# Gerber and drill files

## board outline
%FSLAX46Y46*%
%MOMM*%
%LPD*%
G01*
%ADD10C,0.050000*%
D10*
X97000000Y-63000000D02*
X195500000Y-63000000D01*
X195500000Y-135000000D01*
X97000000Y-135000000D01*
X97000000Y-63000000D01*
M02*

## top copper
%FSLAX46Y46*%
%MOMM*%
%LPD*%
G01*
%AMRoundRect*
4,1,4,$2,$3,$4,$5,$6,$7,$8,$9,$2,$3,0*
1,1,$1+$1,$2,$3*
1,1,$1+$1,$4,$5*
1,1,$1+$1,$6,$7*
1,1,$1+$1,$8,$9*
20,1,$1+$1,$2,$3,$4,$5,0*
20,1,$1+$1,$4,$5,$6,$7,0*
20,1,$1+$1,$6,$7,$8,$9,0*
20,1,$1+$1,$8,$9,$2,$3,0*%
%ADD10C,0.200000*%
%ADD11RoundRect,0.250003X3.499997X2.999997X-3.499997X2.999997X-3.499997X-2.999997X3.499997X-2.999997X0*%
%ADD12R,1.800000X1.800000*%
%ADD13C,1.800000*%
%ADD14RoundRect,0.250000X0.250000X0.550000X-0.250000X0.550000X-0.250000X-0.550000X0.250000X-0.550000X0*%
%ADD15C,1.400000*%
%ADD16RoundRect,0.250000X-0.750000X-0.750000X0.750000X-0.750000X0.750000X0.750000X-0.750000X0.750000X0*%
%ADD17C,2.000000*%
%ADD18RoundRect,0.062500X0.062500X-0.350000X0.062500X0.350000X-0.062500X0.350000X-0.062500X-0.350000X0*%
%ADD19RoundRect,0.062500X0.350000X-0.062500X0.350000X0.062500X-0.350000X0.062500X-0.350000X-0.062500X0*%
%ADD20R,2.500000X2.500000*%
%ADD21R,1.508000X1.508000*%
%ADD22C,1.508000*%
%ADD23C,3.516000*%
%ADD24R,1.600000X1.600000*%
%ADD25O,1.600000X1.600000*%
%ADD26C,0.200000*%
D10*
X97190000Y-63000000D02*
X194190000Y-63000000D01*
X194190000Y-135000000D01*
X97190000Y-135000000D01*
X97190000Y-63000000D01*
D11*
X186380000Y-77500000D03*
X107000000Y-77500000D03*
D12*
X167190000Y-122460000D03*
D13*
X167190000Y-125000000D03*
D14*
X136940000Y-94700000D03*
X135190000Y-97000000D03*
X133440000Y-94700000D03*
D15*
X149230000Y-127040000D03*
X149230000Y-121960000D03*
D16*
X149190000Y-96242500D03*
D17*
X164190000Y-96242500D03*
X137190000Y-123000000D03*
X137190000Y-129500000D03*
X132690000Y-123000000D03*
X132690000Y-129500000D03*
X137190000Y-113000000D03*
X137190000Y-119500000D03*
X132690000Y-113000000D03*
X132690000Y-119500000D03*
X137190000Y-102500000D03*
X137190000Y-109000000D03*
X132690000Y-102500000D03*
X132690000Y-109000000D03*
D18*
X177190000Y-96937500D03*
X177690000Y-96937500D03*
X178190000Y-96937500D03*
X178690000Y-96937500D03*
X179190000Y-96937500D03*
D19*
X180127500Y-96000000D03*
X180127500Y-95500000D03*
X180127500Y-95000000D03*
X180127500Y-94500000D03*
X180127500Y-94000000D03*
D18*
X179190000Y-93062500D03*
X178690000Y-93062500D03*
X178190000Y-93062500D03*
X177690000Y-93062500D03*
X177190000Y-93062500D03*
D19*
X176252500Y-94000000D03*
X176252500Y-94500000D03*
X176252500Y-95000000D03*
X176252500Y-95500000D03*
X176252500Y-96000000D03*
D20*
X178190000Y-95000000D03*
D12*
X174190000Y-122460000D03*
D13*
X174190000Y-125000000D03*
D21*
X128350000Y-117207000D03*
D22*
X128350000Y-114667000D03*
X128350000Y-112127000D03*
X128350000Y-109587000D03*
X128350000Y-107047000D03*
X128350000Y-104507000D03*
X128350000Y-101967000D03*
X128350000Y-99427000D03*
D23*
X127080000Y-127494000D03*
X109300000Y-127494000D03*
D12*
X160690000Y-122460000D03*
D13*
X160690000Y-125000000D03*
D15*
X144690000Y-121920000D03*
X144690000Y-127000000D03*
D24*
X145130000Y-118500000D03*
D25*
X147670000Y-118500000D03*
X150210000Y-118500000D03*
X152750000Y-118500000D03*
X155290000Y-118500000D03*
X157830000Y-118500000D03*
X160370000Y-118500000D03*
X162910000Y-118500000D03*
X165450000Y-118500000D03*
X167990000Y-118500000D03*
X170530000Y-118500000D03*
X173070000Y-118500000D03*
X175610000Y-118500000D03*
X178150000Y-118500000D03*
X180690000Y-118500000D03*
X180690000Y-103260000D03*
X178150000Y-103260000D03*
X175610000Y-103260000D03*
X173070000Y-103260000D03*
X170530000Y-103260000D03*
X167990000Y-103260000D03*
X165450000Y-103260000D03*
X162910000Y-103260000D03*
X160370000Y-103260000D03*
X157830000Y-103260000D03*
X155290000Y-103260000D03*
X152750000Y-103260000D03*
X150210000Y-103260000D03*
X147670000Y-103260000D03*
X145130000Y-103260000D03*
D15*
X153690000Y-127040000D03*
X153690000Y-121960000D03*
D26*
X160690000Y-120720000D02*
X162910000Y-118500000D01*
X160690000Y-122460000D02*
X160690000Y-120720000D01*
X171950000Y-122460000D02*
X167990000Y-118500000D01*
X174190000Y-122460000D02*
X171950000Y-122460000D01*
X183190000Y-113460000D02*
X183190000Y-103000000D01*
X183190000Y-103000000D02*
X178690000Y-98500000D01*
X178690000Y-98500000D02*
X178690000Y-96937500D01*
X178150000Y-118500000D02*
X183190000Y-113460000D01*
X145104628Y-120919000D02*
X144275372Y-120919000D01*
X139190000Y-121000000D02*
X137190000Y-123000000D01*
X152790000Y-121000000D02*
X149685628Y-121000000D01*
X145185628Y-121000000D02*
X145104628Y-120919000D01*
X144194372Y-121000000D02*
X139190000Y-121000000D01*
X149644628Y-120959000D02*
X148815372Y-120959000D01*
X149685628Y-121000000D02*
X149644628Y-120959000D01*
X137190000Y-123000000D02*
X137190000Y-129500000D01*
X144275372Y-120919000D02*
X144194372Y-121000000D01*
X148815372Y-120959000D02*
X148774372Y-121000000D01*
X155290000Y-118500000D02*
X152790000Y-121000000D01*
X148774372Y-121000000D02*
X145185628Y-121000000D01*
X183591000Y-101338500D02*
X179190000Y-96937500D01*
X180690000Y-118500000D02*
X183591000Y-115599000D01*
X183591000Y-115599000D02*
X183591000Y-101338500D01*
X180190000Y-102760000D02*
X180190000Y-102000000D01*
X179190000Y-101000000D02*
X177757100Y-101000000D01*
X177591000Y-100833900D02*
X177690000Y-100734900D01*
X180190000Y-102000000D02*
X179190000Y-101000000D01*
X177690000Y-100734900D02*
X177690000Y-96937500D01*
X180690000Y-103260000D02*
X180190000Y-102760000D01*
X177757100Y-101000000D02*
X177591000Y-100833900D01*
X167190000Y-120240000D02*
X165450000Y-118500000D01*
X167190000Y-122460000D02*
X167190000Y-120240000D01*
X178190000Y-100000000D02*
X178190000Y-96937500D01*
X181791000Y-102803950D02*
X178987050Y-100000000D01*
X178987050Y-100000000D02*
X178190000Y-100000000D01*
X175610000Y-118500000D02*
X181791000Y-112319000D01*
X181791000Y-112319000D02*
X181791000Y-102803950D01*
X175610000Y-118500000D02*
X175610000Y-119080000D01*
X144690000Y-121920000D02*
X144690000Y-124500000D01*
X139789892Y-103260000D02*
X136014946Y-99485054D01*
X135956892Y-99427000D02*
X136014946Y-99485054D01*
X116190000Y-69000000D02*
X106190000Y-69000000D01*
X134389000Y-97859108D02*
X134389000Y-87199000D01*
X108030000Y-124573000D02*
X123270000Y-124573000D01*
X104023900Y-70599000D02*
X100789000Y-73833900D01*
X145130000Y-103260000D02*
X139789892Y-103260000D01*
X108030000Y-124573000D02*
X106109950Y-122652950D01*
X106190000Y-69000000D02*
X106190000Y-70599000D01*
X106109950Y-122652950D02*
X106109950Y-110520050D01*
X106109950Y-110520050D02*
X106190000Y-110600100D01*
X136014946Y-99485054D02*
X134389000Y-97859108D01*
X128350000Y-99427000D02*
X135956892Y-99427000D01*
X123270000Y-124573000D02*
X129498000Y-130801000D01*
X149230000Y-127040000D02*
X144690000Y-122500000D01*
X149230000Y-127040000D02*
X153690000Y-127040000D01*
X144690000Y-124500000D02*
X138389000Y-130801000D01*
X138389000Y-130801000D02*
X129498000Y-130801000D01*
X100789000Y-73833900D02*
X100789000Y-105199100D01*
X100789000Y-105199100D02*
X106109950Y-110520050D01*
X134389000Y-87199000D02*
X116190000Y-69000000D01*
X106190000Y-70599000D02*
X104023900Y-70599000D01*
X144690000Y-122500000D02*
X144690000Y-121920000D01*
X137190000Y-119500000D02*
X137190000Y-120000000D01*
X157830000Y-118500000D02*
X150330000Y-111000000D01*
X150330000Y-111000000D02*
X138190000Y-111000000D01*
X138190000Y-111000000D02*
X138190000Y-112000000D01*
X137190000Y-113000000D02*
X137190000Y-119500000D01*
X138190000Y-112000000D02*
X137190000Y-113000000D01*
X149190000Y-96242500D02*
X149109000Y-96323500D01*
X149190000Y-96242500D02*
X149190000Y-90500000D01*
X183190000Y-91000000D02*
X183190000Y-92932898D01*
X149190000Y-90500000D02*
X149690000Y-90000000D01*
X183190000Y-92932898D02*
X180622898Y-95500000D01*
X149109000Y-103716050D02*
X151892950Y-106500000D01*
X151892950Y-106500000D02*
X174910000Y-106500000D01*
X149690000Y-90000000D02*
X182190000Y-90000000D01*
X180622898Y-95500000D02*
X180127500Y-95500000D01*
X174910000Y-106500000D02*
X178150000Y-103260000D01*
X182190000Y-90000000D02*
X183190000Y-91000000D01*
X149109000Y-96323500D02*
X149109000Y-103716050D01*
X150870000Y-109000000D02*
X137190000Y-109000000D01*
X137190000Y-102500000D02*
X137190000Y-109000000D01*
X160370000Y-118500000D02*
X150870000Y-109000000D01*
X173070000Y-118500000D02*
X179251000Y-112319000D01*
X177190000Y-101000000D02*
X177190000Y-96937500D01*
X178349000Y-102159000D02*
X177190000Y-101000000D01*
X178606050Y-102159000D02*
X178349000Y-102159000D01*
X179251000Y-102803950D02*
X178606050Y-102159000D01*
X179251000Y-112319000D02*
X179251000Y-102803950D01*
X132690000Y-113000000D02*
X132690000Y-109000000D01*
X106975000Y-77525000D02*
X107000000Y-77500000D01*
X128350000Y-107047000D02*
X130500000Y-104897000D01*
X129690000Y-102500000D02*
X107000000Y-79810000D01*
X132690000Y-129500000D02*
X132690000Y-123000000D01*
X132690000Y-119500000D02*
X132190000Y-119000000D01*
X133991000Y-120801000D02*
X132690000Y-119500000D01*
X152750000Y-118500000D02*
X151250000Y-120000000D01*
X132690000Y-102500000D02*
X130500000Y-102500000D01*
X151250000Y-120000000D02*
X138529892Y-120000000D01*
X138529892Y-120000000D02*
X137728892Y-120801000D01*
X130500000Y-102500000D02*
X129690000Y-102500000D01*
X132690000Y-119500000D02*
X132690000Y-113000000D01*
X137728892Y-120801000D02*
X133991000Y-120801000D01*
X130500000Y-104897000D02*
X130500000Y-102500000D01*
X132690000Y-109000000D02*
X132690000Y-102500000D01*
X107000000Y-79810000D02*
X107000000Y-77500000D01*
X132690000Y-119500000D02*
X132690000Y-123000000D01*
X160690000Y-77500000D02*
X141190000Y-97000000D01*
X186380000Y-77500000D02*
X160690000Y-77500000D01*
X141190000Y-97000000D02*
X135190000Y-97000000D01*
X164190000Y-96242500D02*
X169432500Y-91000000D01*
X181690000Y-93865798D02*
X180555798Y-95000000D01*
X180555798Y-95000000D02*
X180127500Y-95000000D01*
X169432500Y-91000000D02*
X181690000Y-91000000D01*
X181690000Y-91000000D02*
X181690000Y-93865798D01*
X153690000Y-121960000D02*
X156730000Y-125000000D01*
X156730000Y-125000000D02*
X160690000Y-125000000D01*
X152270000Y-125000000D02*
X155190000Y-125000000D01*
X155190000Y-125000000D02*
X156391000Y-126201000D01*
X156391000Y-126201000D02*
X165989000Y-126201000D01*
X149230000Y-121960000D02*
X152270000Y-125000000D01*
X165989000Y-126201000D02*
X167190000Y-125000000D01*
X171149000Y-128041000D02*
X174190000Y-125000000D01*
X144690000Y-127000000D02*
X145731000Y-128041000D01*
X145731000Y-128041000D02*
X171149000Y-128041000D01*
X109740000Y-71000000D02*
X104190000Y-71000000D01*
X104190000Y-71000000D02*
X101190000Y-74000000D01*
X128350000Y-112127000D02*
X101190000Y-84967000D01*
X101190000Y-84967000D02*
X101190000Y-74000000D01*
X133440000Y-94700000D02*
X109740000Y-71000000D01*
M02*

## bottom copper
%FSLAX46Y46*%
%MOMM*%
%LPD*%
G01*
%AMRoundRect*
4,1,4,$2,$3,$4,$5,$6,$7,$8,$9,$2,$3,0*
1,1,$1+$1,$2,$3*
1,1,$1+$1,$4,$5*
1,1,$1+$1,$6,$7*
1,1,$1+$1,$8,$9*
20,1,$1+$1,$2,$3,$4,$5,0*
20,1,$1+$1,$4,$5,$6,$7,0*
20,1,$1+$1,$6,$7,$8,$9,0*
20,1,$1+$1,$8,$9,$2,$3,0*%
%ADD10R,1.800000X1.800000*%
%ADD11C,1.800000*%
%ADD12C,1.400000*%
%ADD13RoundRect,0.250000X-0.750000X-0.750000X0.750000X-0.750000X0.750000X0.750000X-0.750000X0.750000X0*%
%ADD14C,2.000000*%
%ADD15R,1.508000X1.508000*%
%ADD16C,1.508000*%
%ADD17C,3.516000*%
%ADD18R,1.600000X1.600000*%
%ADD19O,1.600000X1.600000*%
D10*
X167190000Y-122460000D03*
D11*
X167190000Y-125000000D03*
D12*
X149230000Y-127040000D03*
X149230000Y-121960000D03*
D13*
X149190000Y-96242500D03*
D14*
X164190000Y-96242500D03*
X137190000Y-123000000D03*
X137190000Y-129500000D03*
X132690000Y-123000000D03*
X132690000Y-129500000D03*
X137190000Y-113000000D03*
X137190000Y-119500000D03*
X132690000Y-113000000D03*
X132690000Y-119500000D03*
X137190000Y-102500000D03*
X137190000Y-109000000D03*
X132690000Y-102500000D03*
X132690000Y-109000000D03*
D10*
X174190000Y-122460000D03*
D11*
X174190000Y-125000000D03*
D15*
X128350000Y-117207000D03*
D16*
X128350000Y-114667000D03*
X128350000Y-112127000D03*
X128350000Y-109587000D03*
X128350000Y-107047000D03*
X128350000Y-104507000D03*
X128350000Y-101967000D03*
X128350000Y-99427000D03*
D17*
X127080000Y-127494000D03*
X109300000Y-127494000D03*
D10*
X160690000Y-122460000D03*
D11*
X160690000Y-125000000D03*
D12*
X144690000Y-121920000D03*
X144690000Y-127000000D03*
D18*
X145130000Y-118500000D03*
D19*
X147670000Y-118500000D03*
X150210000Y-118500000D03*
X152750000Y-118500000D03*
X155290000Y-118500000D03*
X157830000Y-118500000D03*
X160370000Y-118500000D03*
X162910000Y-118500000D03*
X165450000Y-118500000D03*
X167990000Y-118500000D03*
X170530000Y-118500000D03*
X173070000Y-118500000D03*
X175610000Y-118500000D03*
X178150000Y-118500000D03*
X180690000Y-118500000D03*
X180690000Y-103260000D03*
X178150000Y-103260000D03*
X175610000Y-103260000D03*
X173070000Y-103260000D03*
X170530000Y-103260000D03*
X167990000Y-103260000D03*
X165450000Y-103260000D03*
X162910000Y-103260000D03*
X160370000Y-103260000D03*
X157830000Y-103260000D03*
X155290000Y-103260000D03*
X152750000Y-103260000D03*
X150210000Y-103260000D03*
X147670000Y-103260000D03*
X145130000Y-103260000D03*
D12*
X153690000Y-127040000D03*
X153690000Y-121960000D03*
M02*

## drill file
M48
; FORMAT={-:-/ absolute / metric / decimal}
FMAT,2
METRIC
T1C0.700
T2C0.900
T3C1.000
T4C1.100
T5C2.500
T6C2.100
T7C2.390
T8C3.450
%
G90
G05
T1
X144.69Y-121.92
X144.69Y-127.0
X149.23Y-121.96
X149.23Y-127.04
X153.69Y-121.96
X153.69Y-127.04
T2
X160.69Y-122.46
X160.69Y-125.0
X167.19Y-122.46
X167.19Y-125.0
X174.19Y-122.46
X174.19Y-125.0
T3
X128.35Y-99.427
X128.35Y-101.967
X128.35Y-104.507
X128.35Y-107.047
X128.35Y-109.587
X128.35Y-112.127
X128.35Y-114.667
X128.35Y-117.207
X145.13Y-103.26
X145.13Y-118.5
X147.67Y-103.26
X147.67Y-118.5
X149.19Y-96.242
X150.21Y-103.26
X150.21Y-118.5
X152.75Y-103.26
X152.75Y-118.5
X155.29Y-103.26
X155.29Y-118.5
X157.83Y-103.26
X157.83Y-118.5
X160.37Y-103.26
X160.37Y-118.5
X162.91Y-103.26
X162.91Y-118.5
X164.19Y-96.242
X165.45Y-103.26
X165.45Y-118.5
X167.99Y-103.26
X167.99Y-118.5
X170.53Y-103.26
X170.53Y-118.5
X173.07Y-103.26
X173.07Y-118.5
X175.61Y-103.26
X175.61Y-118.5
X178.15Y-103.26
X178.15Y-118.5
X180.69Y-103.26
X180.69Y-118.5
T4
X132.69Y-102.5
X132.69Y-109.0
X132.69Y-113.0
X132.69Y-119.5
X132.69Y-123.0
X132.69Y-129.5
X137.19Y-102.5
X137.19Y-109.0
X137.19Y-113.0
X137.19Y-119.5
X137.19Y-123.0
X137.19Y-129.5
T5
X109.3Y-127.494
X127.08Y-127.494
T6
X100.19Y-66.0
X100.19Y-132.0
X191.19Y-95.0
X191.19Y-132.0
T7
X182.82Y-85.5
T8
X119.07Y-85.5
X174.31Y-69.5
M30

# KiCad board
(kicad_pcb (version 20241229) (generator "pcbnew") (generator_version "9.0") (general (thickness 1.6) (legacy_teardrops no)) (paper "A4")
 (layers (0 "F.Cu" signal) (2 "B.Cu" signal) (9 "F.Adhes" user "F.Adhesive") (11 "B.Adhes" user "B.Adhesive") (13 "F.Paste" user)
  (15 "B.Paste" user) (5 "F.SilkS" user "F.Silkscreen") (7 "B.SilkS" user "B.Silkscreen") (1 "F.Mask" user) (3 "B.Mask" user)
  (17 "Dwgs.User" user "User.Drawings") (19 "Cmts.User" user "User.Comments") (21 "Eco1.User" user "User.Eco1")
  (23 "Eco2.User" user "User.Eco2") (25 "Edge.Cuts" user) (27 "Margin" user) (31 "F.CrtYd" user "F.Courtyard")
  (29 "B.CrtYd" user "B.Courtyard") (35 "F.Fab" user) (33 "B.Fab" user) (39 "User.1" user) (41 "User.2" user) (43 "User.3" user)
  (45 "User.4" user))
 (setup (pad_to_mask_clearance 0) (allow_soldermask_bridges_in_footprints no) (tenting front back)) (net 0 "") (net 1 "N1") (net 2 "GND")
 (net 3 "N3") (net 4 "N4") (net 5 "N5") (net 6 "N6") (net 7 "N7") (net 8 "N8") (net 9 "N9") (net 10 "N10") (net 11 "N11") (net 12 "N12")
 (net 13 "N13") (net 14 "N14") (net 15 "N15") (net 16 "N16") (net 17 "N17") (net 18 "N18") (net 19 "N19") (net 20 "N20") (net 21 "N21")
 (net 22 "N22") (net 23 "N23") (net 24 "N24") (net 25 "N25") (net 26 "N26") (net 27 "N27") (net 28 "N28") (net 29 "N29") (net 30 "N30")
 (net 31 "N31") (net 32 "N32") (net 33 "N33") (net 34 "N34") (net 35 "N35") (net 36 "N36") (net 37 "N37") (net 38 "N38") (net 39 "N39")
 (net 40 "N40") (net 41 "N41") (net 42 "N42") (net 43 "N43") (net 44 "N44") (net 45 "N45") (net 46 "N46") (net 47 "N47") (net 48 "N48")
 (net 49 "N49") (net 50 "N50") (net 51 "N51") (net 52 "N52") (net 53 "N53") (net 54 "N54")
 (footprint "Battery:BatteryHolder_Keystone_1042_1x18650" (layer "F.Cu") (at 146.69 77.5 180)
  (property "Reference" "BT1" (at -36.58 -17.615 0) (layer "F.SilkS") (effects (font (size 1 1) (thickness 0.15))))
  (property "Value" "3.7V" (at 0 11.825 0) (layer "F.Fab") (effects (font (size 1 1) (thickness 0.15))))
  (pad "" np_thru_hole circle (at -36.13 -8 180) (size 2.39 2.39) (drill 2.39) (layers "*.Cu" "*.Mask"))
  (pad "" np_thru_hole circle (at -27.62 8 180) (size 3.45 3.45) (drill 3.45) (layers "*.Cu" "*.Mask"))
  (pad "" np_thru_hole circle (at 27.62 -8 180) (size 3.45 3.45) (drill 3.45) (layers "*.Cu" "*.Mask"))
  (pad "1" smd roundrect (at -39.69 0 180) (size 7.5 6.5) (layers "F.Cu" "F.Mask" "F.Paste") (roundrect_rratio 0.038462) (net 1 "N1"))
  (pad "2" smd roundrect (at 39.69 0 180) (size 7.5 6.5) (layers "F.Cu" "F.Mask" "F.Paste") (roundrect_rratio 0.038462) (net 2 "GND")))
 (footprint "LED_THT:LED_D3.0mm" (layer "F.Cu") (at 167.19 122.46 -90)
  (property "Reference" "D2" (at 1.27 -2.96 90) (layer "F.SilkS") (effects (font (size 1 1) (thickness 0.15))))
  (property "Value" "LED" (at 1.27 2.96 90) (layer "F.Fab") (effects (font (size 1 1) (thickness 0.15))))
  (pad "1" thru_hole rect (at 0 0 270) (size 1.8 1.8) (drill 0.9) (layers "*.Cu" "*.Mask") (remove_unused_layers no) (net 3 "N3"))
  (pad "2" thru_hole circle (at 2.54 0 270) (size 1.8 1.8) (drill 0.9) (layers "*.Cu" "*.Mask") (remove_unused_layers no) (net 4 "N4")))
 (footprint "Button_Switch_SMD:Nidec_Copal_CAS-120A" (layer "F.Cu") (at 135.19 95.85 -90)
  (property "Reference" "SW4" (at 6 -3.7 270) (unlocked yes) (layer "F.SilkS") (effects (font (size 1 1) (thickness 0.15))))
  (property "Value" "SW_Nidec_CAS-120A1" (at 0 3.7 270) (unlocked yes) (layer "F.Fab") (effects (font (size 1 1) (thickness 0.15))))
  (pad "1" smd roundrect (at -1.15 -1.75 180) (size 1 1.6) (layers "F.Cu" "F.Mask" "F.Paste") (roundrect_rratio 0.25) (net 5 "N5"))
  (pad "2" smd roundrect (at 1.15 0 180) (size 1 1.6) (layers "F.Cu" "F.Mask" "F.Paste") (roundrect_rratio 0.25) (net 1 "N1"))
  (pad "3" smd roundrect (at -1.15 1.75 180) (size 1 1.6) (layers "F.Cu" "F.Mask" "F.Paste") (roundrect_rratio 0.25) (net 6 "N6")))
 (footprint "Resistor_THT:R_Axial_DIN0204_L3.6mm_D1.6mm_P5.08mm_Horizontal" (layer "F.Cu") (at 149.23 127.04 90)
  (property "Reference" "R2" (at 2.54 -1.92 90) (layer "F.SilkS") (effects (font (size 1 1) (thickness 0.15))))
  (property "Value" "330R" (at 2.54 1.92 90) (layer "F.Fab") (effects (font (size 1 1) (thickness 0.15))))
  (pad "1" thru_hole circle (at 0 0 90) (size 1.4 1.4) (drill 0.7) (layers "*.Cu" "*.Mask") (remove_unused_layers no) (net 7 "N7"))
  (pad "2" thru_hole circle (at 5.08 0 90) (size 1.4 1.4) (drill 0.7) (layers "*.Cu" "*.Mask") (remove_unused_layers no) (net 4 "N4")))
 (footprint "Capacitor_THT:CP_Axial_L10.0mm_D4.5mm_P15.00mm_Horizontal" (layer "F.Cu") (at 149.19 96.2425)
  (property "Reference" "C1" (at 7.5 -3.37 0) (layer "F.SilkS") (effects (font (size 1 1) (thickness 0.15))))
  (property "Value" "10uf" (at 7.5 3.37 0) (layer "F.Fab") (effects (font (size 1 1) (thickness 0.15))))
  (pad "1" thru_hole roundrect (at 0 0) (size 2 2) (drill 1) (layers "*.Cu" "*.Mask") (remove_unused_layers no) (roundrect_rratio 0.125)
   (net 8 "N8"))
  (pad "2" thru_hole circle (at 15 0) (size 2 2) (drill 1) (layers "*.Cu" "*.Mask") (remove_unused_layers no) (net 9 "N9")))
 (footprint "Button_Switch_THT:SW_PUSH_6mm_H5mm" (layer "F.Cu") (at 137.19 123 -90)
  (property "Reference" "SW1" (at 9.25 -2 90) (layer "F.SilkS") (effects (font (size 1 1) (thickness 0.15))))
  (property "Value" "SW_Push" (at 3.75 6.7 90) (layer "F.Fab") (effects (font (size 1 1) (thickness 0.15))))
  (pad "1" thru_hole circle (at 0 0) (size 2 2) (drill 1.1) (layers "*.Cu" "*.Mask") (remove_unused_layers no) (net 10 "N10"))
  (pad "1" thru_hole circle (at 6.5 0) (size 2 2) (drill 1.1) (layers "*.Cu" "*.Mask") (remove_unused_layers no) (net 10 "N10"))
  (pad "2" thru_hole circle (at 0 4.5) (size 2 2) (drill 1.1) (layers "*.Cu" "*.Mask") (remove_unused_layers no) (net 2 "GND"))
  (pad "2" thru_hole circle (at 6.5 4.5) (size 2 2) (drill 1.1) (layers "*.Cu" "*.Mask") (remove_unused_layers no) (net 2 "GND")))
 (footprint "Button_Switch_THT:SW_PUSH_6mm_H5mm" (layer "F.Cu") (at 137.19 113 -90)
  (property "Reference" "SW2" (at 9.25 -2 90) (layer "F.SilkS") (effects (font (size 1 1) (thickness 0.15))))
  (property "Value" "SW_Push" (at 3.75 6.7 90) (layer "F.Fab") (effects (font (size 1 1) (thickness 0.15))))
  (pad "1" thru_hole circle (at 0 0) (size 2 2) (drill 1.1) (layers "*.Cu" "*.Mask") (remove_unused_layers no) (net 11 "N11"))
  (pad "1" thru_hole circle (at 6.5 0) (size 2 2) (drill 1.1) (layers "*.Cu" "*.Mask") (remove_unused_layers no) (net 11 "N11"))
  (pad "2" thru_hole circle (at 0 4.5) (size 2 2) (drill 1.1) (layers "*.Cu" "*.Mask") (remove_unused_layers no) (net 2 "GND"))
  (pad "2" thru_hole circle (at 6.5 4.5) (size 2 2) (drill 1.1) (layers "*.Cu" "*.Mask") (remove_unused_layers no) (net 2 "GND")))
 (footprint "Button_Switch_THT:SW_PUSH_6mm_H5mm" (layer "F.Cu") (at 137.19 102.5 -90)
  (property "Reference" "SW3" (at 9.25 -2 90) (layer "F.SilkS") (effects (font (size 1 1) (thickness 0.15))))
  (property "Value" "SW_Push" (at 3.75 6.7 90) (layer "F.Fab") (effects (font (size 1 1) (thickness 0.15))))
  (pad "1" thru_hole circle (at 0 0) (size 2 2) (drill 1.1) (layers "*.Cu" "*.Mask") (remove_unused_layers no) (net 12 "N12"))
  (pad "1" thru_hole circle (at 6.5 0) (size 2 2) (drill 1.1) (layers "*.Cu" "*.Mask") (remove_unused_layers no) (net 12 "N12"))
  (pad "2" thru_hole circle (at 0 4.5) (size 2 2) (drill 1.1) (layers "*.Cu" "*.Mask") (remove_unused_layers no) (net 2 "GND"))
  (pad "2" thru_hole circle (at 6.5 4.5) (size 2 2) (drill 1.1) (layers "*.Cu" "*.Mask") (remove_unused_layers no) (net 2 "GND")))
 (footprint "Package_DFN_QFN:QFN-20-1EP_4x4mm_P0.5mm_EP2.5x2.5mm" (layer "F.Cu") (at 178.19 95 90)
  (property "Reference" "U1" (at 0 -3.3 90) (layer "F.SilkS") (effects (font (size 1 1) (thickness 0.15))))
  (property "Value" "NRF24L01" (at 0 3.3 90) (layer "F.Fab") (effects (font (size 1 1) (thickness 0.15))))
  (pad "" smd roundrect (at -0.625 -0.625 90) (size 1.01 1.01) (layers "F.Paste") (roundrect_rratio 0.247525))
  (pad "" smd roundrect (at -0.625 0.625 90) (size 1.01 1.01) (layers "F.Paste") (roundrect_rratio 0.247525))
  (pad "" smd roundrect (at 0.625 -0.625 90) (size 1.01 1.01) (layers "F.Paste") (roundrect_rratio 0.247525))
  (pad "" smd roundrect (at 0.625 0.625 90) (size 1.01 1.01) (layers "F.Paste") (roundrect_rratio 0.247525))
  (pad "1" smd roundrect (at -1.9375 -1 90) (size 0.825 0.25) (layers "F.Cu" "F.Mask" "F.Paste") (roundrect_rratio 0.25) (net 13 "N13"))
  (pad "2" smd roundrect (at -1.9375 -0.5 90) (size 0.825 0.25) (layers "F.Cu" "F.Mask" "F.Paste") (roundrect_rratio 0.25) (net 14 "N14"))
  (pad "3" smd roundrect (at -1.9375 0 90) (size 0.825 0.25) (layers "F.Cu" "F.Mask" "F.Paste") (roundrect_rratio 0.25) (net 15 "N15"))
  (pad "4" smd roundrect (at -1.9375 0.5 90) (size 0.825 0.25) (layers "F.Cu" "F.Mask" "F.Paste") (roundrect_rratio 0.25) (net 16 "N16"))
  (pad "5" smd roundrect (at -1.9375 1 90) (size 0.825 0.25) (layers "F.Cu" "F.Mask" "F.Paste") (roundrect_rratio 0.25) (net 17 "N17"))
  (pad "6" smd roundrect (at -1 1.9375 90) (size 0.25 0.825) (layers "F.Cu" "F.Mask" "F.Paste") (roundrect_rratio 0.25) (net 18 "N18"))
  (pad "7" smd roundrect (at -0.5 1.9375 90) (size 0.25 0.825) (layers "F.Cu" "F.Mask" "F.Paste") (roundrect_rratio 0.25) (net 8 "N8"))
  (pad "8" smd roundrect (at 0 1.9375 90) (size 0.25 0.825) (layers "F.Cu" "F.Mask" "F.Paste") (roundrect_rratio 0.25) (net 9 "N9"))
  (pad "9" smd roundrect (at 0.5 1.9375 90) (size 0.25 0.825) (layers "F.Cu" "F.Mask" "F.Paste") (roundrect_rratio 0.25) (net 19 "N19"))
  (pad "10" smd roundrect (at 1 1.9375 90) (size 0.25 0.825) (layers "F.Cu" "F.Mask" "F.Paste") (roundrect_rratio 0.25) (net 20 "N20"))
  (pad "11" smd roundrect (at 1.9375 1 90) (size 0.825 0.25) (layers "F.Cu" "F.Mask" "F.Paste") (roundrect_rratio 0.25) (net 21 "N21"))
  (pad "12" smd roundrect (at 1.9375 0.5 90) (size 0.825 0.25) (layers "F.Cu" "F.Mask" "F.Paste") (roundrect_rratio 0.25) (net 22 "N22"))
  (pad "13" smd roundrect (at 1.9375 0 90) (size 0.825 0.25) (layers "F.Cu" "F.Mask" "F.Paste") (roundrect_rratio 0.25) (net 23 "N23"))
  (pad "14" smd roundrect (at 1.9375 -0.5 90) (size 0.825 0.25) (layers "F.Cu" "F.Mask" "F.Paste") (roundrect_rratio 0.25) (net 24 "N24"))
  (pad "15" smd roundrect (at 1.9375 -1 90) (size 0.825 0.25) (layers "F.Cu" "F.Mask" "F.Paste") (roundrect_rratio 0.25) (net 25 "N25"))
  (pad "16" smd roundrect (at 1 -1.9375 90) (size 0.25 0.825) (layers "F.Cu" "F.Mask" "F.Paste") (roundrect_rratio 0.25) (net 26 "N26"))
  (pad "17" smd roundrect (at 0.5 -1.9375 90) (size 0.25 0.825) (layers "F.Cu" "F.Mask" "F.Paste") (roundrect_rratio 0.25) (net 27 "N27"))
  (pad "18" smd roundrect (at 0 -1.9375 90) (size 0.25 0.825) (layers "F.Cu" "F.Mask" "F.Paste") (roundrect_rratio 0.25) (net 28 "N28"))
  (pad "19" smd roundrect (at -0.5 -1.9375 90) (size 0.25 0.825) (layers "F.Cu" "F.Mask" "F.Paste") (roundrect_rratio 0.25) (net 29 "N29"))
  (pad "20" smd roundrect (at -1 -1.9375 90) (size 0.25 0.825) (layers "F.Cu" "F.Mask" "F.Paste") (roundrect_rratio 0.25) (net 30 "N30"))
  (pad "21" smd rect (at 0 0 90) (size 2.5 2.5) (layers "F.Cu" "F.Mask") (zone_connect 2)))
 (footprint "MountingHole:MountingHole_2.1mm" (layer "F.Cu") (at 191.19 95 -90)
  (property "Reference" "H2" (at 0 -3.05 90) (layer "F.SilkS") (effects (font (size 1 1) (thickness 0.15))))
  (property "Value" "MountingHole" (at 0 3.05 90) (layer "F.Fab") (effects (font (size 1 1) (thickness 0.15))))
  (pad "" np_thru_hole circle (at 0 0 270) (size 2.1 2.1) (drill 2.1) (layers "*.Cu" "*.Mask")))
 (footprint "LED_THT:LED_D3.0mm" (layer "F.Cu") (at 174.19 122.46 -90)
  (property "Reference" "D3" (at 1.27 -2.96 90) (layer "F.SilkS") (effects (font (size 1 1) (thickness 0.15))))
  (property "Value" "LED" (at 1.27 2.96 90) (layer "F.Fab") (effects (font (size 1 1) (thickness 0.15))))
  (pad "1" thru_hole rect (at 0 0 270) (size 1.8 1.8) (drill 0.9) (layers "*.Cu" "*.Mask") (remove_unused_layers no) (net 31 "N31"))
  (pad "2" thru_hole circle (at 2.54 0 270) (size 1.8 1.8) (drill 0.9) (layers "*.Cu" "*.Mask") (remove_unused_layers no) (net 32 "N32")))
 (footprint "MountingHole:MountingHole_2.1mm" (layer "F.Cu") (at 100.19 66 -90)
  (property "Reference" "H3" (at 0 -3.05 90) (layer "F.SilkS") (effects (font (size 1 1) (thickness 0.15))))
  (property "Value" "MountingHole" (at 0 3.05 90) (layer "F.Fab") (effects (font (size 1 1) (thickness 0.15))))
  (pad "" np_thru_hole circle (at 0 0 270) (size 2.1 2.1) (drill 2.1) (layers "*.Cu" "*.Mask")))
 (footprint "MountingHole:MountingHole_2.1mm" (layer "F.Cu") (at 191.19 132 -90)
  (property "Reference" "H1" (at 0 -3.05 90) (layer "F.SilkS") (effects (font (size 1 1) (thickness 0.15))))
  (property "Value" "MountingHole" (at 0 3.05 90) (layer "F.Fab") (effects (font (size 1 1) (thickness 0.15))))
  (pad "" np_thru_hole circle (at 0 0 270) (size 2.1 2.1) (drill 2.1) (layers "*.Cu" "*.Mask")))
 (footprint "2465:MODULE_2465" (layer "F.Cu") (at 118.19 112 90)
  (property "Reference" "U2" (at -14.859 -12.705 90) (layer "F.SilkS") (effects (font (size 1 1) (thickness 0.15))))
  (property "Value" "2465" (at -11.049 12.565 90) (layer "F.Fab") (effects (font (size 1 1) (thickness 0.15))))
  (pad "1" thru_hole rect (at -5.207 10.16 90) (size 1.508 1.508) (drill 1) (layers "*.Cu" "*.Mask") (remove_unused_layers no)
   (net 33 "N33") (solder_mask_margin 0.102))
  (pad "2" thru_hole circle (at -2.667 10.16 90) (size 1.508 1.508) (drill 1) (layers "*.Cu" "*.Mask") (remove_unused_layers no)
   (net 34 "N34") (solder_mask_margin 0.102))
  (pad "3" thru_hole circle (at -0.127 10.16 90) (size 1.508 1.508) (drill 1) (layers "*.Cu" "*.Mask") (remove_unused_layers no)
   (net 6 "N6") (solder_mask_margin 0.102))
  (pad "4" thru_hole circle (at 2.413 10.16 90) (size 1.508 1.508) (drill 1) (layers "*.Cu" "*.Mask") (remove_unused_layers no)
   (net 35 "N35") (solder_mask_margin 0.102))
  (pad "5" thru_hole circle (at 4.953 10.16 90) (size 1.508 1.508) (drill 1) (layers "*.Cu" "*.Mask") (remove_unused_layers no)
   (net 2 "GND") (solder_mask_margin 0.102))
  (pad "6" thru_hole circle (at 7.493 10.16 90) (size 1.508 1.508) (drill 1) (layers "*.Cu" "*.Mask") (remove_unused_layers no)
   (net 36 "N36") (solder_mask_margin 0.102))
  (pad "7" thru_hole circle (at 10.033 10.16 90) (size 1.508 1.508) (drill 1) (layers "*.Cu" "*.Mask") (remove_unused_layers no)
   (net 2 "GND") (solder_mask_margin 0.102))
  (pad "8" thru_hole circle (at 12.573 10.16 90) (size 1.508 1.508) (drill 1) (layers "*.Cu" "*.Mask") (remove_unused_layers no)
   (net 7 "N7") (solder_mask_margin 0.102))
  (pad "P1" thru_hole circle (at -15.494 8.89 90) (size 3.516 3.516) (drill 2.5) (layers "*.Cu" "*.Mask") (remove_unused_layers no)
   (solder_mask_margin 0.102))
  (pad "P2" thru_hole circle (at -15.494 -8.89 90) (size 3.516 3.516) (drill 2.5) (layers "*.Cu" "*.Mask") (remove_unused_layers no)
   (solder_mask_margin 0.102)))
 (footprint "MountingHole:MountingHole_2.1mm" (layer "F.Cu") (at 100.19 132 -90)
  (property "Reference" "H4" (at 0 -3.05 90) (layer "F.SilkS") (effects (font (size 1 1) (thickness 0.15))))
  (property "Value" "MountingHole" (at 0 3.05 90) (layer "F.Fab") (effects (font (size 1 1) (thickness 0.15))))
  (pad "" np_thru_hole circle (at 0 0 270) (size 2.1 2.1) (drill 2.1) (layers "*.Cu" "*.Mask")))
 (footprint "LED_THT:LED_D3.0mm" (layer "F.Cu") (at 160.69 122.46 -90)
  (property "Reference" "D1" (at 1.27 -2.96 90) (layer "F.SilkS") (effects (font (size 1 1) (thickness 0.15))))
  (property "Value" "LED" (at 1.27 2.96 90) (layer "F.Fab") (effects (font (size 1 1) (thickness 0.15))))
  (pad "1" thru_hole rect (at 0 0 270) (size 1.8 1.8) (drill 0.9) (layers "*.Cu" "*.Mask") (remove_unused_layers no) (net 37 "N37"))
  (pad "2" thru_hole circle (at 2.54 0 270) (size 1.8 1.8) (drill 0.9) (layers "*.Cu" "*.Mask") (remove_unused_layers no) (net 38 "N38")))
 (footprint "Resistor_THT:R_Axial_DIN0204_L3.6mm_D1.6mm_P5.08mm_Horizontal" (layer "F.Cu") (at 144.69 121.92 -90)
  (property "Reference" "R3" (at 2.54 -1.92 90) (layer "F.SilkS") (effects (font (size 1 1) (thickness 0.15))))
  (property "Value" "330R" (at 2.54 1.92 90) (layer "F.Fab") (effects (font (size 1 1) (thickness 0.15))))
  (pad "1" thru_hole circle (at 0 0 270) (size 1.4 1.4) (drill 0.7) (layers "*.Cu" "*.Mask") (remove_unused_layers no) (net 7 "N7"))
  (pad "2" thru_hole circle (at 5.08 0 270) (size 1.4 1.4) (drill 0.7) (layers "*.Cu" "*.Mask") (remove_unused_layers no) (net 32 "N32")))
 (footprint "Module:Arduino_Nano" (layer "F.Cu") (at 145.13 118.5 90)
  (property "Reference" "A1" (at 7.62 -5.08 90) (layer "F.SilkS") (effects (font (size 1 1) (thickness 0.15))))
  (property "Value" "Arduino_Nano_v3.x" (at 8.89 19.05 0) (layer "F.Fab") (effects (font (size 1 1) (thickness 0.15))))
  (pad "1" thru_hole rect (at 0 0 90) (size 1.6 1.6) (drill 1) (layers "*.Cu" "*.Mask") (remove_unused_layers no) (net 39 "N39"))
  (pad "2" thru_hole oval (at 0 2.54 90) (size 1.6 1.6) (drill 1) (layers "*.Cu" "*.Mask") (remove_unused_layers no) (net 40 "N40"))
  (pad "3" thru_hole oval (at 0 5.08 90) (size 1.6 1.6) (drill 1) (layers "*.Cu" "*.Mask") (remove_unused_layers no) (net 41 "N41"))
  (pad "4" thru_hole oval (at 0 7.62 90) (size 1.6 1.6) (drill 1) (layers "*.Cu" "*.Mask") (remove_unused_layers no) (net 2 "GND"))
  (pad "5" thru_hole oval (at 0 10.16 90) (size 1.6 1.6) (drill 1) (layers "*.Cu" "*.Mask") (remove_unused_layers no) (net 10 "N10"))
  (pad "6" thru_hole oval (at 0 12.7 90) (size 1.6 1.6) (drill 1) (layers "*.Cu" "*.Mask") (remove_unused_layers no) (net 11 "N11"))
  (pad "7" thru_hole oval (at 0 15.24 90) (size 1.6 1.6) (drill 1) (layers "*.Cu" "*.Mask") (remove_unused_layers no) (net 12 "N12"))
  (pad "8" thru_hole oval (at 0 17.78 90) (size 1.6 1.6) (drill 1) (layers "*.Cu" "*.Mask") (remove_unused_layers no) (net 37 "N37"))
  (pad "9" thru_hole oval (at 0 20.32 90) (size 1.6 1.6) (drill 1) (layers "*.Cu" "*.Mask") (remove_unused_layers no) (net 3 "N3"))
  (pad "10" thru_hole oval (at 0 22.86 90) (size 1.6 1.6) (drill 1) (layers "*.Cu" "*.Mask") (remove_unused_layers no) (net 31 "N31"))
  (pad "11" thru_hole oval (at 0 25.4 90) (size 1.6 1.6) (drill 1) (layers "*.Cu" "*.Mask") (remove_unused_layers no) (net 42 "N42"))
  (pad "12" thru_hole oval (at 0 27.94 90) (size 1.6 1.6) (drill 1) (layers "*.Cu" "*.Mask") (remove_unused_layers no) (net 13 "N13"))
  (pad "13" thru_hole oval (at 0 30.48 90) (size 1.6 1.6) (drill 1) (layers "*.Cu" "*.Mask") (remove_unused_layers no) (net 15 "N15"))
  (pad "14" thru_hole oval (at 0 33.02 90) (size 1.6 1.6) (drill 1) (layers "*.Cu" "*.Mask") (remove_unused_layers no) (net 16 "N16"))
  (pad "15" thru_hole oval (at 0 35.56 90) (size 1.6 1.6) (drill 1) (layers "*.Cu" "*.Mask") (remove_unused_layers no) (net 17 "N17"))
  (pad "16" thru_hole oval (at 15.24 35.56 90) (size 1.6 1.6) (drill 1) (layers "*.Cu" "*.Mask") (remove_unused_layers no) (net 14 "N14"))
  (pad "17" thru_hole oval (at 15.24 33.02 90) (size 1.6 1.6) (drill 1) (layers "*.Cu" "*.Mask") (remove_unused_layers no) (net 8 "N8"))
  (pad "18" thru_hole oval (at 15.24 30.48 90) (size 1.6 1.6) (drill 1) (layers "*.Cu" "*.Mask") (remove_unused_layers no) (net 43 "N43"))
  (pad "19" thru_hole oval (at 15.24 27.94 90) (size 1.6 1.6) (drill 1) (layers "*.Cu" "*.Mask") (remove_unused_layers no) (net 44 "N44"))
  (pad "20" thru_hole oval (at 15.24 25.4 90) (size 1.6 1.6) (drill 1) (layers "*.Cu" "*.Mask") (remove_unused_layers no) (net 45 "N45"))
  (pad "21" thru_hole oval (at 15.24 22.86 90) (size 1.6 1.6) (drill 1) (layers "*.Cu" "*.Mask") (remove_unused_layers no) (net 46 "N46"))
  (pad "22" thru_hole oval (at 15.24 20.32 90) (size 1.6 1.6) (drill 1) (layers "*.Cu" "*.Mask") (remove_unused_layers no) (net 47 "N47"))
  (pad "23" thru_hole oval (at 15.24 17.78 90) (size 1.6 1.6) (drill 1) (layers "*.Cu" "*.Mask") (remove_unused_layers no) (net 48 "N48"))
  (pad "24" thru_hole oval (at 15.24 15.24 90) (size 1.6 1.6) (drill 1) (layers "*.Cu" "*.Mask") (remove_unused_layers no) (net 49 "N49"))
  (pad "25" thru_hole oval (at 15.24 12.7 90) (size 1.6 1.6) (drill 1) (layers "*.Cu" "*.Mask") (remove_unused_layers no) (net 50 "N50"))
  (pad "26" thru_hole oval (at 15.24 10.16 90) (size 1.6 1.6) (drill 1) (layers "*.Cu" "*.Mask") (remove_unused_layers no) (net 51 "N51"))
  (pad "27" thru_hole oval (at 15.24 7.62 90) (size 1.6 1.6) (drill 1) (layers "*.Cu" "*.Mask") (remove_unused_layers no) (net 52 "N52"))
  (pad "28" thru_hole oval (at 15.24 5.08 90) (size 1.6 1.6) (drill 1) (layers "*.Cu" "*.Mask") (remove_unused_layers no) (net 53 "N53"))
  (pad "29" thru_hole oval (at 15.24 2.54 90) (size 1.6 1.6) (drill 1) (layers "*.Cu" "*.Mask") (remove_unused_layers no) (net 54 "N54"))
  (pad "30" thru_hole oval (at 15.24 0 90) (size 1.6 1.6) (drill 1) (layers "*.Cu" "*.Mask") (remove_unused_layers no) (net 7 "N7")))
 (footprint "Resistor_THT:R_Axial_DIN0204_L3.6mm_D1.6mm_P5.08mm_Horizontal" (layer "F.Cu") (at 153.69 127.04 90)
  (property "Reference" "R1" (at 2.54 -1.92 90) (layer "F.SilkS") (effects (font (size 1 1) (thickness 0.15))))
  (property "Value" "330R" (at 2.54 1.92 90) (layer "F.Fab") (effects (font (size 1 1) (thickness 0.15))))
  (pad "1" thru_hole circle (at 0 0 90) (size 1.4 1.4) (drill 0.7) (layers "*.Cu" "*.Mask") (remove_unused_layers no) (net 7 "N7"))
  (pad "2" thru_hole circle (at 5.08 0 90) (size 1.4 1.4) (drill 0.7) (layers "*.Cu" "*.Mask") (remove_unused_layers no) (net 38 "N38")))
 (gr_rect (start 97.19 63) (end 194.19 135) (stroke (width 0.2) (type default)) (fill no) (layer "F.Cu"))
 (gr_rect (start 97 63) (end 195.5 135) (stroke (width 0.05) (type default)) (fill no) (layer "Edge.Cuts"))
 (segment (start 160.69 120.72) (end 162.91 118.5) (width 0.2) (layer "F.Cu") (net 37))
 (segment (start 160.69 122.46) (end 160.69 120.72) (width 0.2) (layer "F.Cu") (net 37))
 (segment (start 171.95 122.46) (end 167.99 118.5) (width 0.2) (layer "F.Cu") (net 31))
 (segment (start 174.19 122.46) (end 171.95 122.46) (width 0.2) (layer "F.Cu") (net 31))
 (segment (start 183.19 113.46) (end 183.19 103) (width 0.2) (layer "F.Cu") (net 16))
 (segment (start 183.19 103) (end 178.69 98.5) (width 0.2) (layer "F.Cu") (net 16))
 (segment (start 178.69 98.5) (end 178.69 96.9375) (width 0.2) (layer "F.Cu") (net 16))
 (segment (start 178.15 118.5) (end 183.19 113.46) (width 0.2) (layer "F.Cu") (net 16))
 (segment (start 145.104628 120.919) (end 144.275372 120.919) (width 0.2) (layer "F.Cu") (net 10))
 (segment (start 139.19 121) (end 137.19 123) (width 0.2) (layer "F.Cu") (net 10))
 (segment (start 152.79 121) (end 149.685628 121) (width 0.2) (layer "F.Cu") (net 10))
 (segment (start 145.185628 121) (end 145.104628 120.919) (width 0.2) (layer "F.Cu") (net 10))
 (segment (start 144.194372 121) (end 139.19 121) (width 0.2) (layer "F.Cu") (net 10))
 (segment (start 149.644628 120.959) (end 148.815372 120.959) (width 0.2) (layer "F.Cu") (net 10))
 (segment (start 149.685628 121) (end 149.644628 120.959) (width 0.2) (layer "F.Cu") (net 10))
 (segment (start 137.19 123) (end 137.19 129.5) (width 0.2) (layer "F.Cu") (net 10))
 (segment (start 144.275372 120.919) (end 144.194372 121) (width 0.2) (layer "F.Cu") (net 10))
 (segment (start 148.815372 120.959) (end 148.774372 121) (width 0.2) (layer "F.Cu") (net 10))
 (segment (start 155.29 118.5) (end 152.79 121) (width 0.2) (layer "F.Cu") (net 10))
 (segment (start 148.774372 121) (end 145.185628 121) (width 0.2) (layer "F.Cu") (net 10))
 (segment (start 183.591 101.3385) (end 179.19 96.9375) (width 0.2) (layer "F.Cu") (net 17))
 (segment (start 180.69 118.5) (end 183.591 115.599) (width 0.2) (layer "F.Cu") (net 17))
 (segment (start 183.591 115.599) (end 183.591 101.3385) (width 0.2) (layer "F.Cu") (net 17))
 (segment (start 180.19 102.76) (end 180.19 102) (width 0.2) (layer "F.Cu") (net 14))
 (segment (start 179.19 101) (end 177.7571 101) (width 0.2) (layer "F.Cu") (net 14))
 (segment (start 177.591 100.8339) (end 177.69 100.7349) (width 0.2) (layer "F.Cu") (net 14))
 (segment (start 180.19 102) (end 179.19 101) (width 0.2) (layer "F.Cu") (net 14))
 (segment (start 177.69 100.7349) (end 177.69 96.9375) (width 0.2) (layer "F.Cu") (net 14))
 (segment (start 180.69 103.26) (end 180.19 102.76) (width 0.2) (layer "F.Cu") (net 14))
 (segment (start 177.7571 101) (end 177.591 100.8339) (width 0.2) (layer "F.Cu") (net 14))
 (segment (start 167.19 120.24) (end 165.45 118.5) (width 0.2) (layer "F.Cu") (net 3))
 (segment (start 167.19 122.46) (end 167.19 120.24) (width 0.2) (layer "F.Cu") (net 3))
 (segment (start 178.19 100) (end 178.19 96.9375) (width 0.2) (layer "F.Cu") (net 15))
 (segment (start 181.791 102.80395) (end 178.98705 100) (width 0.2) (layer "F.Cu") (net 15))
 (segment (start 178.98705 100) (end 178.19 100) (width 0.2) (layer "F.Cu") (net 15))
 (segment (start 175.61 118.5) (end 181.791 112.319) (width 0.2) (layer "F.Cu") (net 15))
 (segment (start 181.791 112.319) (end 181.791 102.80395) (width 0.2) (layer "F.Cu") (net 15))
 (segment (start 175.61 118.5) (end 175.61 119.08) (width 0.2) (layer "F.Cu") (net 15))
 (segment (start 144.69 121.92) (end 144.69 124.5) (width 0.2) (layer "F.Cu") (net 7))
 (segment (start 139.789892 103.26) (end 136.014946 99.485054) (width 0.2) (layer "F.Cu") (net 7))
 (segment (start 135.956892 99.427) (end 136.014946 99.485054) (width 0.2) (layer "F.Cu") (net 7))
 (segment (start 116.19 69) (end 106.19 69) (width 0.2) (layer "F.Cu") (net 7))
 (segment (start 134.389 97.859108) (end 134.389 87.199) (width 0.2) (layer "F.Cu") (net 7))
 (segment (start 108.03 124.573) (end 123.27 124.573) (width 0.2) (layer "F.Cu") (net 7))
 (segment (start 104.0239 70.599) (end 100.789 73.8339) (width 0.2) (layer "F.Cu") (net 7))
 (segment (start 145.13 103.26) (end 139.789892 103.26) (width 0.2) (layer "F.Cu") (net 7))
 (segment (start 108.03 124.573) (end 106.10995 122.65295) (width 0.2) (layer "F.Cu") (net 7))
 (segment (start 106.19 69) (end 106.19 70.599) (width 0.2) (layer "F.Cu") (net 7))
 (segment (start 106.10995 122.65295) (end 106.10995 110.52005) (width 0.2) (layer "F.Cu") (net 7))
 (segment (start 106.10995 110.52005) (end 106.19 110.6001) (width 0.2) (layer "F.Cu") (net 7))
 (segment (start 136.014946 99.485054) (end 134.389 97.859108) (width 0.2) (layer "F.Cu") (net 7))
 (segment (start 128.35 99.427) (end 135.956892 99.427) (width 0.2) (layer "F.Cu") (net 7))
 (segment (start 123.27 124.573) (end 129.498 130.801) (width 0.2) (layer "F.Cu") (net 7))
 (segment (start 149.23 127.04) (end 144.69 122.5) (width 0.2) (layer "F.Cu") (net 7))
 (segment (start 149.23 127.04) (end 153.69 127.04) (width 0.2) (layer "F.Cu") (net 7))
 (segment (start 144.69 124.5) (end 138.389 130.801) (width 0.2) (layer "F.Cu") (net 7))
 (segment (start 138.389 130.801) (end 129.498 130.801) (width 0.2) (layer "F.Cu") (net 7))
 (segment (start 100.789 73.8339) (end 100.789 105.1991) (width 0.2) (layer "F.Cu") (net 7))
 (segment (start 100.789 105.1991) (end 106.10995 110.52005) (width 0.2) (layer "F.Cu") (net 7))
 (segment (start 134.389 87.199) (end 116.19 69) (width 0.2) (layer "F.Cu") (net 7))
 (segment (start 106.19 70.599) (end 104.0239 70.599) (width 0.2) (layer "F.Cu") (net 7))
 (segment (start 144.69 122.5) (end 144.69 121.92) (width 0.2) (layer "F.Cu") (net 7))
 (segment (start 137.19 119.5) (end 137.19 120) (width 0.2) (layer "F.Cu") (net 11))
 (segment (start 157.83 118.5) (end 150.33 111) (width 0.2) (layer "F.Cu") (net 11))
 (segment (start 150.33 111) (end 138.19 111) (width 0.2) (layer "F.Cu") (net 11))
 (segment (start 138.19 111) (end 138.19 112) (width 0.2) (layer "F.Cu") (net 11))
 (segment (start 137.19 113) (end 137.19 119.5) (width 0.2) (layer "F.Cu") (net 11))
 (segment (start 138.19 112) (end 137.19 113) (width 0.2) (layer "F.Cu") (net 11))
 (segment (start 149.19 96.2425) (end 149.109 96.3235) (width 0.2) (layer "F.Cu") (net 8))
 (segment (start 149.19 96.2425) (end 149.19 90.5) (width 0.2) (layer "F.Cu") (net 8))
 (segment (start 183.19 91) (end 183.19 92.932898) (width 0.2) (layer "F.Cu") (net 8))
 (segment (start 149.19 90.5) (end 149.69 90) (width 0.2) (layer "F.Cu") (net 8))
 (segment (start 183.19 92.932898) (end 180.622898 95.5) (width 0.2) (layer "F.Cu") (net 8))
 (segment (start 149.109 103.71605) (end 151.89295 106.5) (width 0.2) (layer "F.Cu") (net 8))
 (segment (start 151.89295 106.5) (end 174.91 106.5) (width 0.2) (layer "F.Cu") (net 8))
 (segment (start 149.69 90) (end 182.19 90) (width 0.2) (layer "F.Cu") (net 8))
 (segment (start 180.622898 95.5) (end 180.1275 95.5) (width 0.2) (layer "F.Cu") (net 8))
 (segment (start 174.91 106.5) (end 178.15 103.26) (width 0.2) (layer "F.Cu") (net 8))
 (segment (start 182.19 90) (end 183.19 91) (width 0.2) (layer "F.Cu") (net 8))
 (segment (start 149.109 96.3235) (end 149.109 103.71605) (width 0.2) (layer "F.Cu") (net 8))
 (segment (start 150.87 109) (end 137.19 109) (width 0.2) (layer "F.Cu") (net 12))
 (segment (start 137.19 102.5) (end 137.19 109) (width 0.2) (layer "F.Cu") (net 12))
 (segment (start 160.37 118.5) (end 150.87 109) (width 0.2) (layer "F.Cu") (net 12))
 (segment (start 173.07 118.5) (end 179.251 112.319) (width 0.2) (layer "F.Cu") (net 13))
 (segment (start 177.19 101) (end 177.19 96.9375) (width 0.2) (layer "F.Cu") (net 13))
 (segment (start 178.349 102.159) (end 177.19 101) (width 0.2) (layer "F.Cu") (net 13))
 (segment (start 178.60605 102.159) (end 178.349 102.159) (width 0.2) (layer "F.Cu") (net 13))
 (segment (start 179.251 102.80395) (end 178.60605 102.159) (width 0.2) (layer "F.Cu") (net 13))
 (segment (start 179.251 112.319) (end 179.251 102.80395) (width 0.2) (layer "F.Cu") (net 13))
 (segment (start 132.69 113) (end 132.69 109) (width 0.2) (layer "F.Cu") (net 2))
 (segment (start 106.975 77.525) (end 107 77.5) (width 0.2) (layer "F.Cu") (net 2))
 (segment (start 128.35 107.047) (end 130.5 104.897) (width 0.2) (layer "F.Cu") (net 2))
 (segment (start 129.69 102.5) (end 107 79.81) (width 0.2) (layer "F.Cu") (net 2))
 (segment (start 132.69 129.5) (end 132.69 123) (width 0.2) (layer "F.Cu") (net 2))
 (segment (start 132.69 119.5) (end 132.19 119) (width 0.2) (layer "F.Cu") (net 2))
 (segment (start 133.991 120.801) (end 132.69 119.5) (width 0.2) (layer "F.Cu") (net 2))
 (segment (start 152.75 118.5) (end 151.25 120) (width 0.2) (layer "F.Cu") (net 2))
 (segment (start 132.69 102.5) (end 130.5 102.5) (width 0.2) (layer "F.Cu") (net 2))
 (segment (start 151.25 120) (end 138.529892 120) (width 0.2) (layer "F.Cu") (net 2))
 (segment (start 138.529892 120) (end 137.728892 120.801) (width 0.2) (layer "F.Cu") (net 2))
 (segment (start 130.5 102.5) (end 129.69 102.5) (width 0.2) (layer "F.Cu") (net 2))
 (segment (start 132.69 119.5) (end 132.69 113) (width 0.2) (layer "F.Cu") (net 2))
 (segment (start 137.728892 120.801) (end 133.991 120.801) (width 0.2) (layer "F.Cu") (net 2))
 (segment (start 130.5 104.897) (end 130.5 102.5) (width 0.2) (layer "F.Cu") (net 2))
 (segment (start 132.69 109) (end 132.69 102.5) (width 0.2) (layer "F.Cu") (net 2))
 (segment (start 107 79.81) (end 107 77.5) (width 0.2) (layer "F.Cu") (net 2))
 (segment (start 132.69 119.5) (end 132.69 123) (width 0.2) (layer "F.Cu") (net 2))
 (segment (start 160.69 77.5) (end 141.19 97) (width 0.2) (layer "F.Cu") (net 1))
 (segment (start 186.38 77.5) (end 160.69 77.5) (width 0.2) (layer "F.Cu") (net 1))
 (segment (start 141.19 97) (end 135.19 97) (width 0.2) (layer "F.Cu") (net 1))
 (segment (start 164.19 96.2425) (end 169.4325 91) (width 0.2) (layer "F.Cu") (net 9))
 (segment (start 181.69 93.865798) (end 180.555798 95) (width 0.2) (layer "F.Cu") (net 9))
 (segment (start 180.555798 95) (end 180.1275 95) (width 0.2) (layer "F.Cu") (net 9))
 (segment (start 169.4325 91) (end 181.69 91) (width 0.2) (layer "F.Cu") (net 9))
 (segment (start 181.69 91) (end 181.69 93.865798) (width 0.2) (layer "F.Cu") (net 9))
 (segment (start 153.69 121.96) (end 156.73 125) (width 0.2) (layer "F.Cu") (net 38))
 (segment (start 156.73 125) (end 160.69 125) (width 0.2) (layer "F.Cu") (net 38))
 (segment (start 152.27 125) (end 155.19 125) (width 0.2) (layer "F.Cu") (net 4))
 (segment (start 155.19 125) (end 156.391 126.201) (width 0.2) (layer "F.Cu") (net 4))
 (segment (start 156.391 126.201) (end 165.989 126.201) (width 0.2) (layer "F.Cu") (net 4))
 (segment (start 149.23 121.96) (end 152.27 125) (width 0.2) (layer "F.Cu") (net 4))
 (segment (start 165.989 126.201) (end 167.19 125) (width 0.2) (layer "F.Cu") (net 4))
 (segment (start 171.149 128.041) (end 174.19 125) (width 0.2) (layer "F.Cu") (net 32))
 (segment (start 144.69 127) (end 145.731 128.041) (width 0.2) (layer "F.Cu") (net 32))
 (segment (start 145.731 128.041) (end 171.149 128.041) (width 0.2) (layer "F.Cu") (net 32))
 (segment (start 109.74 71) (end 104.19 71) (width 0.2) (layer "F.Cu") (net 6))
 (segment (start 104.19 71) (end 101.19 74) (width 0.2) (layer "F.Cu") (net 6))
 (segment (start 128.35 112.127) (end 101.19 84.967) (width 0.2) (layer "F.Cu") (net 6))
 (segment (start 101.19 84.967) (end 101.19 74) (width 0.2) (layer "F.Cu") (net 6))
 (segment (start 133.44 94.7) (end 109.74 71) (width 0.2) (layer "F.Cu") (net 6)))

